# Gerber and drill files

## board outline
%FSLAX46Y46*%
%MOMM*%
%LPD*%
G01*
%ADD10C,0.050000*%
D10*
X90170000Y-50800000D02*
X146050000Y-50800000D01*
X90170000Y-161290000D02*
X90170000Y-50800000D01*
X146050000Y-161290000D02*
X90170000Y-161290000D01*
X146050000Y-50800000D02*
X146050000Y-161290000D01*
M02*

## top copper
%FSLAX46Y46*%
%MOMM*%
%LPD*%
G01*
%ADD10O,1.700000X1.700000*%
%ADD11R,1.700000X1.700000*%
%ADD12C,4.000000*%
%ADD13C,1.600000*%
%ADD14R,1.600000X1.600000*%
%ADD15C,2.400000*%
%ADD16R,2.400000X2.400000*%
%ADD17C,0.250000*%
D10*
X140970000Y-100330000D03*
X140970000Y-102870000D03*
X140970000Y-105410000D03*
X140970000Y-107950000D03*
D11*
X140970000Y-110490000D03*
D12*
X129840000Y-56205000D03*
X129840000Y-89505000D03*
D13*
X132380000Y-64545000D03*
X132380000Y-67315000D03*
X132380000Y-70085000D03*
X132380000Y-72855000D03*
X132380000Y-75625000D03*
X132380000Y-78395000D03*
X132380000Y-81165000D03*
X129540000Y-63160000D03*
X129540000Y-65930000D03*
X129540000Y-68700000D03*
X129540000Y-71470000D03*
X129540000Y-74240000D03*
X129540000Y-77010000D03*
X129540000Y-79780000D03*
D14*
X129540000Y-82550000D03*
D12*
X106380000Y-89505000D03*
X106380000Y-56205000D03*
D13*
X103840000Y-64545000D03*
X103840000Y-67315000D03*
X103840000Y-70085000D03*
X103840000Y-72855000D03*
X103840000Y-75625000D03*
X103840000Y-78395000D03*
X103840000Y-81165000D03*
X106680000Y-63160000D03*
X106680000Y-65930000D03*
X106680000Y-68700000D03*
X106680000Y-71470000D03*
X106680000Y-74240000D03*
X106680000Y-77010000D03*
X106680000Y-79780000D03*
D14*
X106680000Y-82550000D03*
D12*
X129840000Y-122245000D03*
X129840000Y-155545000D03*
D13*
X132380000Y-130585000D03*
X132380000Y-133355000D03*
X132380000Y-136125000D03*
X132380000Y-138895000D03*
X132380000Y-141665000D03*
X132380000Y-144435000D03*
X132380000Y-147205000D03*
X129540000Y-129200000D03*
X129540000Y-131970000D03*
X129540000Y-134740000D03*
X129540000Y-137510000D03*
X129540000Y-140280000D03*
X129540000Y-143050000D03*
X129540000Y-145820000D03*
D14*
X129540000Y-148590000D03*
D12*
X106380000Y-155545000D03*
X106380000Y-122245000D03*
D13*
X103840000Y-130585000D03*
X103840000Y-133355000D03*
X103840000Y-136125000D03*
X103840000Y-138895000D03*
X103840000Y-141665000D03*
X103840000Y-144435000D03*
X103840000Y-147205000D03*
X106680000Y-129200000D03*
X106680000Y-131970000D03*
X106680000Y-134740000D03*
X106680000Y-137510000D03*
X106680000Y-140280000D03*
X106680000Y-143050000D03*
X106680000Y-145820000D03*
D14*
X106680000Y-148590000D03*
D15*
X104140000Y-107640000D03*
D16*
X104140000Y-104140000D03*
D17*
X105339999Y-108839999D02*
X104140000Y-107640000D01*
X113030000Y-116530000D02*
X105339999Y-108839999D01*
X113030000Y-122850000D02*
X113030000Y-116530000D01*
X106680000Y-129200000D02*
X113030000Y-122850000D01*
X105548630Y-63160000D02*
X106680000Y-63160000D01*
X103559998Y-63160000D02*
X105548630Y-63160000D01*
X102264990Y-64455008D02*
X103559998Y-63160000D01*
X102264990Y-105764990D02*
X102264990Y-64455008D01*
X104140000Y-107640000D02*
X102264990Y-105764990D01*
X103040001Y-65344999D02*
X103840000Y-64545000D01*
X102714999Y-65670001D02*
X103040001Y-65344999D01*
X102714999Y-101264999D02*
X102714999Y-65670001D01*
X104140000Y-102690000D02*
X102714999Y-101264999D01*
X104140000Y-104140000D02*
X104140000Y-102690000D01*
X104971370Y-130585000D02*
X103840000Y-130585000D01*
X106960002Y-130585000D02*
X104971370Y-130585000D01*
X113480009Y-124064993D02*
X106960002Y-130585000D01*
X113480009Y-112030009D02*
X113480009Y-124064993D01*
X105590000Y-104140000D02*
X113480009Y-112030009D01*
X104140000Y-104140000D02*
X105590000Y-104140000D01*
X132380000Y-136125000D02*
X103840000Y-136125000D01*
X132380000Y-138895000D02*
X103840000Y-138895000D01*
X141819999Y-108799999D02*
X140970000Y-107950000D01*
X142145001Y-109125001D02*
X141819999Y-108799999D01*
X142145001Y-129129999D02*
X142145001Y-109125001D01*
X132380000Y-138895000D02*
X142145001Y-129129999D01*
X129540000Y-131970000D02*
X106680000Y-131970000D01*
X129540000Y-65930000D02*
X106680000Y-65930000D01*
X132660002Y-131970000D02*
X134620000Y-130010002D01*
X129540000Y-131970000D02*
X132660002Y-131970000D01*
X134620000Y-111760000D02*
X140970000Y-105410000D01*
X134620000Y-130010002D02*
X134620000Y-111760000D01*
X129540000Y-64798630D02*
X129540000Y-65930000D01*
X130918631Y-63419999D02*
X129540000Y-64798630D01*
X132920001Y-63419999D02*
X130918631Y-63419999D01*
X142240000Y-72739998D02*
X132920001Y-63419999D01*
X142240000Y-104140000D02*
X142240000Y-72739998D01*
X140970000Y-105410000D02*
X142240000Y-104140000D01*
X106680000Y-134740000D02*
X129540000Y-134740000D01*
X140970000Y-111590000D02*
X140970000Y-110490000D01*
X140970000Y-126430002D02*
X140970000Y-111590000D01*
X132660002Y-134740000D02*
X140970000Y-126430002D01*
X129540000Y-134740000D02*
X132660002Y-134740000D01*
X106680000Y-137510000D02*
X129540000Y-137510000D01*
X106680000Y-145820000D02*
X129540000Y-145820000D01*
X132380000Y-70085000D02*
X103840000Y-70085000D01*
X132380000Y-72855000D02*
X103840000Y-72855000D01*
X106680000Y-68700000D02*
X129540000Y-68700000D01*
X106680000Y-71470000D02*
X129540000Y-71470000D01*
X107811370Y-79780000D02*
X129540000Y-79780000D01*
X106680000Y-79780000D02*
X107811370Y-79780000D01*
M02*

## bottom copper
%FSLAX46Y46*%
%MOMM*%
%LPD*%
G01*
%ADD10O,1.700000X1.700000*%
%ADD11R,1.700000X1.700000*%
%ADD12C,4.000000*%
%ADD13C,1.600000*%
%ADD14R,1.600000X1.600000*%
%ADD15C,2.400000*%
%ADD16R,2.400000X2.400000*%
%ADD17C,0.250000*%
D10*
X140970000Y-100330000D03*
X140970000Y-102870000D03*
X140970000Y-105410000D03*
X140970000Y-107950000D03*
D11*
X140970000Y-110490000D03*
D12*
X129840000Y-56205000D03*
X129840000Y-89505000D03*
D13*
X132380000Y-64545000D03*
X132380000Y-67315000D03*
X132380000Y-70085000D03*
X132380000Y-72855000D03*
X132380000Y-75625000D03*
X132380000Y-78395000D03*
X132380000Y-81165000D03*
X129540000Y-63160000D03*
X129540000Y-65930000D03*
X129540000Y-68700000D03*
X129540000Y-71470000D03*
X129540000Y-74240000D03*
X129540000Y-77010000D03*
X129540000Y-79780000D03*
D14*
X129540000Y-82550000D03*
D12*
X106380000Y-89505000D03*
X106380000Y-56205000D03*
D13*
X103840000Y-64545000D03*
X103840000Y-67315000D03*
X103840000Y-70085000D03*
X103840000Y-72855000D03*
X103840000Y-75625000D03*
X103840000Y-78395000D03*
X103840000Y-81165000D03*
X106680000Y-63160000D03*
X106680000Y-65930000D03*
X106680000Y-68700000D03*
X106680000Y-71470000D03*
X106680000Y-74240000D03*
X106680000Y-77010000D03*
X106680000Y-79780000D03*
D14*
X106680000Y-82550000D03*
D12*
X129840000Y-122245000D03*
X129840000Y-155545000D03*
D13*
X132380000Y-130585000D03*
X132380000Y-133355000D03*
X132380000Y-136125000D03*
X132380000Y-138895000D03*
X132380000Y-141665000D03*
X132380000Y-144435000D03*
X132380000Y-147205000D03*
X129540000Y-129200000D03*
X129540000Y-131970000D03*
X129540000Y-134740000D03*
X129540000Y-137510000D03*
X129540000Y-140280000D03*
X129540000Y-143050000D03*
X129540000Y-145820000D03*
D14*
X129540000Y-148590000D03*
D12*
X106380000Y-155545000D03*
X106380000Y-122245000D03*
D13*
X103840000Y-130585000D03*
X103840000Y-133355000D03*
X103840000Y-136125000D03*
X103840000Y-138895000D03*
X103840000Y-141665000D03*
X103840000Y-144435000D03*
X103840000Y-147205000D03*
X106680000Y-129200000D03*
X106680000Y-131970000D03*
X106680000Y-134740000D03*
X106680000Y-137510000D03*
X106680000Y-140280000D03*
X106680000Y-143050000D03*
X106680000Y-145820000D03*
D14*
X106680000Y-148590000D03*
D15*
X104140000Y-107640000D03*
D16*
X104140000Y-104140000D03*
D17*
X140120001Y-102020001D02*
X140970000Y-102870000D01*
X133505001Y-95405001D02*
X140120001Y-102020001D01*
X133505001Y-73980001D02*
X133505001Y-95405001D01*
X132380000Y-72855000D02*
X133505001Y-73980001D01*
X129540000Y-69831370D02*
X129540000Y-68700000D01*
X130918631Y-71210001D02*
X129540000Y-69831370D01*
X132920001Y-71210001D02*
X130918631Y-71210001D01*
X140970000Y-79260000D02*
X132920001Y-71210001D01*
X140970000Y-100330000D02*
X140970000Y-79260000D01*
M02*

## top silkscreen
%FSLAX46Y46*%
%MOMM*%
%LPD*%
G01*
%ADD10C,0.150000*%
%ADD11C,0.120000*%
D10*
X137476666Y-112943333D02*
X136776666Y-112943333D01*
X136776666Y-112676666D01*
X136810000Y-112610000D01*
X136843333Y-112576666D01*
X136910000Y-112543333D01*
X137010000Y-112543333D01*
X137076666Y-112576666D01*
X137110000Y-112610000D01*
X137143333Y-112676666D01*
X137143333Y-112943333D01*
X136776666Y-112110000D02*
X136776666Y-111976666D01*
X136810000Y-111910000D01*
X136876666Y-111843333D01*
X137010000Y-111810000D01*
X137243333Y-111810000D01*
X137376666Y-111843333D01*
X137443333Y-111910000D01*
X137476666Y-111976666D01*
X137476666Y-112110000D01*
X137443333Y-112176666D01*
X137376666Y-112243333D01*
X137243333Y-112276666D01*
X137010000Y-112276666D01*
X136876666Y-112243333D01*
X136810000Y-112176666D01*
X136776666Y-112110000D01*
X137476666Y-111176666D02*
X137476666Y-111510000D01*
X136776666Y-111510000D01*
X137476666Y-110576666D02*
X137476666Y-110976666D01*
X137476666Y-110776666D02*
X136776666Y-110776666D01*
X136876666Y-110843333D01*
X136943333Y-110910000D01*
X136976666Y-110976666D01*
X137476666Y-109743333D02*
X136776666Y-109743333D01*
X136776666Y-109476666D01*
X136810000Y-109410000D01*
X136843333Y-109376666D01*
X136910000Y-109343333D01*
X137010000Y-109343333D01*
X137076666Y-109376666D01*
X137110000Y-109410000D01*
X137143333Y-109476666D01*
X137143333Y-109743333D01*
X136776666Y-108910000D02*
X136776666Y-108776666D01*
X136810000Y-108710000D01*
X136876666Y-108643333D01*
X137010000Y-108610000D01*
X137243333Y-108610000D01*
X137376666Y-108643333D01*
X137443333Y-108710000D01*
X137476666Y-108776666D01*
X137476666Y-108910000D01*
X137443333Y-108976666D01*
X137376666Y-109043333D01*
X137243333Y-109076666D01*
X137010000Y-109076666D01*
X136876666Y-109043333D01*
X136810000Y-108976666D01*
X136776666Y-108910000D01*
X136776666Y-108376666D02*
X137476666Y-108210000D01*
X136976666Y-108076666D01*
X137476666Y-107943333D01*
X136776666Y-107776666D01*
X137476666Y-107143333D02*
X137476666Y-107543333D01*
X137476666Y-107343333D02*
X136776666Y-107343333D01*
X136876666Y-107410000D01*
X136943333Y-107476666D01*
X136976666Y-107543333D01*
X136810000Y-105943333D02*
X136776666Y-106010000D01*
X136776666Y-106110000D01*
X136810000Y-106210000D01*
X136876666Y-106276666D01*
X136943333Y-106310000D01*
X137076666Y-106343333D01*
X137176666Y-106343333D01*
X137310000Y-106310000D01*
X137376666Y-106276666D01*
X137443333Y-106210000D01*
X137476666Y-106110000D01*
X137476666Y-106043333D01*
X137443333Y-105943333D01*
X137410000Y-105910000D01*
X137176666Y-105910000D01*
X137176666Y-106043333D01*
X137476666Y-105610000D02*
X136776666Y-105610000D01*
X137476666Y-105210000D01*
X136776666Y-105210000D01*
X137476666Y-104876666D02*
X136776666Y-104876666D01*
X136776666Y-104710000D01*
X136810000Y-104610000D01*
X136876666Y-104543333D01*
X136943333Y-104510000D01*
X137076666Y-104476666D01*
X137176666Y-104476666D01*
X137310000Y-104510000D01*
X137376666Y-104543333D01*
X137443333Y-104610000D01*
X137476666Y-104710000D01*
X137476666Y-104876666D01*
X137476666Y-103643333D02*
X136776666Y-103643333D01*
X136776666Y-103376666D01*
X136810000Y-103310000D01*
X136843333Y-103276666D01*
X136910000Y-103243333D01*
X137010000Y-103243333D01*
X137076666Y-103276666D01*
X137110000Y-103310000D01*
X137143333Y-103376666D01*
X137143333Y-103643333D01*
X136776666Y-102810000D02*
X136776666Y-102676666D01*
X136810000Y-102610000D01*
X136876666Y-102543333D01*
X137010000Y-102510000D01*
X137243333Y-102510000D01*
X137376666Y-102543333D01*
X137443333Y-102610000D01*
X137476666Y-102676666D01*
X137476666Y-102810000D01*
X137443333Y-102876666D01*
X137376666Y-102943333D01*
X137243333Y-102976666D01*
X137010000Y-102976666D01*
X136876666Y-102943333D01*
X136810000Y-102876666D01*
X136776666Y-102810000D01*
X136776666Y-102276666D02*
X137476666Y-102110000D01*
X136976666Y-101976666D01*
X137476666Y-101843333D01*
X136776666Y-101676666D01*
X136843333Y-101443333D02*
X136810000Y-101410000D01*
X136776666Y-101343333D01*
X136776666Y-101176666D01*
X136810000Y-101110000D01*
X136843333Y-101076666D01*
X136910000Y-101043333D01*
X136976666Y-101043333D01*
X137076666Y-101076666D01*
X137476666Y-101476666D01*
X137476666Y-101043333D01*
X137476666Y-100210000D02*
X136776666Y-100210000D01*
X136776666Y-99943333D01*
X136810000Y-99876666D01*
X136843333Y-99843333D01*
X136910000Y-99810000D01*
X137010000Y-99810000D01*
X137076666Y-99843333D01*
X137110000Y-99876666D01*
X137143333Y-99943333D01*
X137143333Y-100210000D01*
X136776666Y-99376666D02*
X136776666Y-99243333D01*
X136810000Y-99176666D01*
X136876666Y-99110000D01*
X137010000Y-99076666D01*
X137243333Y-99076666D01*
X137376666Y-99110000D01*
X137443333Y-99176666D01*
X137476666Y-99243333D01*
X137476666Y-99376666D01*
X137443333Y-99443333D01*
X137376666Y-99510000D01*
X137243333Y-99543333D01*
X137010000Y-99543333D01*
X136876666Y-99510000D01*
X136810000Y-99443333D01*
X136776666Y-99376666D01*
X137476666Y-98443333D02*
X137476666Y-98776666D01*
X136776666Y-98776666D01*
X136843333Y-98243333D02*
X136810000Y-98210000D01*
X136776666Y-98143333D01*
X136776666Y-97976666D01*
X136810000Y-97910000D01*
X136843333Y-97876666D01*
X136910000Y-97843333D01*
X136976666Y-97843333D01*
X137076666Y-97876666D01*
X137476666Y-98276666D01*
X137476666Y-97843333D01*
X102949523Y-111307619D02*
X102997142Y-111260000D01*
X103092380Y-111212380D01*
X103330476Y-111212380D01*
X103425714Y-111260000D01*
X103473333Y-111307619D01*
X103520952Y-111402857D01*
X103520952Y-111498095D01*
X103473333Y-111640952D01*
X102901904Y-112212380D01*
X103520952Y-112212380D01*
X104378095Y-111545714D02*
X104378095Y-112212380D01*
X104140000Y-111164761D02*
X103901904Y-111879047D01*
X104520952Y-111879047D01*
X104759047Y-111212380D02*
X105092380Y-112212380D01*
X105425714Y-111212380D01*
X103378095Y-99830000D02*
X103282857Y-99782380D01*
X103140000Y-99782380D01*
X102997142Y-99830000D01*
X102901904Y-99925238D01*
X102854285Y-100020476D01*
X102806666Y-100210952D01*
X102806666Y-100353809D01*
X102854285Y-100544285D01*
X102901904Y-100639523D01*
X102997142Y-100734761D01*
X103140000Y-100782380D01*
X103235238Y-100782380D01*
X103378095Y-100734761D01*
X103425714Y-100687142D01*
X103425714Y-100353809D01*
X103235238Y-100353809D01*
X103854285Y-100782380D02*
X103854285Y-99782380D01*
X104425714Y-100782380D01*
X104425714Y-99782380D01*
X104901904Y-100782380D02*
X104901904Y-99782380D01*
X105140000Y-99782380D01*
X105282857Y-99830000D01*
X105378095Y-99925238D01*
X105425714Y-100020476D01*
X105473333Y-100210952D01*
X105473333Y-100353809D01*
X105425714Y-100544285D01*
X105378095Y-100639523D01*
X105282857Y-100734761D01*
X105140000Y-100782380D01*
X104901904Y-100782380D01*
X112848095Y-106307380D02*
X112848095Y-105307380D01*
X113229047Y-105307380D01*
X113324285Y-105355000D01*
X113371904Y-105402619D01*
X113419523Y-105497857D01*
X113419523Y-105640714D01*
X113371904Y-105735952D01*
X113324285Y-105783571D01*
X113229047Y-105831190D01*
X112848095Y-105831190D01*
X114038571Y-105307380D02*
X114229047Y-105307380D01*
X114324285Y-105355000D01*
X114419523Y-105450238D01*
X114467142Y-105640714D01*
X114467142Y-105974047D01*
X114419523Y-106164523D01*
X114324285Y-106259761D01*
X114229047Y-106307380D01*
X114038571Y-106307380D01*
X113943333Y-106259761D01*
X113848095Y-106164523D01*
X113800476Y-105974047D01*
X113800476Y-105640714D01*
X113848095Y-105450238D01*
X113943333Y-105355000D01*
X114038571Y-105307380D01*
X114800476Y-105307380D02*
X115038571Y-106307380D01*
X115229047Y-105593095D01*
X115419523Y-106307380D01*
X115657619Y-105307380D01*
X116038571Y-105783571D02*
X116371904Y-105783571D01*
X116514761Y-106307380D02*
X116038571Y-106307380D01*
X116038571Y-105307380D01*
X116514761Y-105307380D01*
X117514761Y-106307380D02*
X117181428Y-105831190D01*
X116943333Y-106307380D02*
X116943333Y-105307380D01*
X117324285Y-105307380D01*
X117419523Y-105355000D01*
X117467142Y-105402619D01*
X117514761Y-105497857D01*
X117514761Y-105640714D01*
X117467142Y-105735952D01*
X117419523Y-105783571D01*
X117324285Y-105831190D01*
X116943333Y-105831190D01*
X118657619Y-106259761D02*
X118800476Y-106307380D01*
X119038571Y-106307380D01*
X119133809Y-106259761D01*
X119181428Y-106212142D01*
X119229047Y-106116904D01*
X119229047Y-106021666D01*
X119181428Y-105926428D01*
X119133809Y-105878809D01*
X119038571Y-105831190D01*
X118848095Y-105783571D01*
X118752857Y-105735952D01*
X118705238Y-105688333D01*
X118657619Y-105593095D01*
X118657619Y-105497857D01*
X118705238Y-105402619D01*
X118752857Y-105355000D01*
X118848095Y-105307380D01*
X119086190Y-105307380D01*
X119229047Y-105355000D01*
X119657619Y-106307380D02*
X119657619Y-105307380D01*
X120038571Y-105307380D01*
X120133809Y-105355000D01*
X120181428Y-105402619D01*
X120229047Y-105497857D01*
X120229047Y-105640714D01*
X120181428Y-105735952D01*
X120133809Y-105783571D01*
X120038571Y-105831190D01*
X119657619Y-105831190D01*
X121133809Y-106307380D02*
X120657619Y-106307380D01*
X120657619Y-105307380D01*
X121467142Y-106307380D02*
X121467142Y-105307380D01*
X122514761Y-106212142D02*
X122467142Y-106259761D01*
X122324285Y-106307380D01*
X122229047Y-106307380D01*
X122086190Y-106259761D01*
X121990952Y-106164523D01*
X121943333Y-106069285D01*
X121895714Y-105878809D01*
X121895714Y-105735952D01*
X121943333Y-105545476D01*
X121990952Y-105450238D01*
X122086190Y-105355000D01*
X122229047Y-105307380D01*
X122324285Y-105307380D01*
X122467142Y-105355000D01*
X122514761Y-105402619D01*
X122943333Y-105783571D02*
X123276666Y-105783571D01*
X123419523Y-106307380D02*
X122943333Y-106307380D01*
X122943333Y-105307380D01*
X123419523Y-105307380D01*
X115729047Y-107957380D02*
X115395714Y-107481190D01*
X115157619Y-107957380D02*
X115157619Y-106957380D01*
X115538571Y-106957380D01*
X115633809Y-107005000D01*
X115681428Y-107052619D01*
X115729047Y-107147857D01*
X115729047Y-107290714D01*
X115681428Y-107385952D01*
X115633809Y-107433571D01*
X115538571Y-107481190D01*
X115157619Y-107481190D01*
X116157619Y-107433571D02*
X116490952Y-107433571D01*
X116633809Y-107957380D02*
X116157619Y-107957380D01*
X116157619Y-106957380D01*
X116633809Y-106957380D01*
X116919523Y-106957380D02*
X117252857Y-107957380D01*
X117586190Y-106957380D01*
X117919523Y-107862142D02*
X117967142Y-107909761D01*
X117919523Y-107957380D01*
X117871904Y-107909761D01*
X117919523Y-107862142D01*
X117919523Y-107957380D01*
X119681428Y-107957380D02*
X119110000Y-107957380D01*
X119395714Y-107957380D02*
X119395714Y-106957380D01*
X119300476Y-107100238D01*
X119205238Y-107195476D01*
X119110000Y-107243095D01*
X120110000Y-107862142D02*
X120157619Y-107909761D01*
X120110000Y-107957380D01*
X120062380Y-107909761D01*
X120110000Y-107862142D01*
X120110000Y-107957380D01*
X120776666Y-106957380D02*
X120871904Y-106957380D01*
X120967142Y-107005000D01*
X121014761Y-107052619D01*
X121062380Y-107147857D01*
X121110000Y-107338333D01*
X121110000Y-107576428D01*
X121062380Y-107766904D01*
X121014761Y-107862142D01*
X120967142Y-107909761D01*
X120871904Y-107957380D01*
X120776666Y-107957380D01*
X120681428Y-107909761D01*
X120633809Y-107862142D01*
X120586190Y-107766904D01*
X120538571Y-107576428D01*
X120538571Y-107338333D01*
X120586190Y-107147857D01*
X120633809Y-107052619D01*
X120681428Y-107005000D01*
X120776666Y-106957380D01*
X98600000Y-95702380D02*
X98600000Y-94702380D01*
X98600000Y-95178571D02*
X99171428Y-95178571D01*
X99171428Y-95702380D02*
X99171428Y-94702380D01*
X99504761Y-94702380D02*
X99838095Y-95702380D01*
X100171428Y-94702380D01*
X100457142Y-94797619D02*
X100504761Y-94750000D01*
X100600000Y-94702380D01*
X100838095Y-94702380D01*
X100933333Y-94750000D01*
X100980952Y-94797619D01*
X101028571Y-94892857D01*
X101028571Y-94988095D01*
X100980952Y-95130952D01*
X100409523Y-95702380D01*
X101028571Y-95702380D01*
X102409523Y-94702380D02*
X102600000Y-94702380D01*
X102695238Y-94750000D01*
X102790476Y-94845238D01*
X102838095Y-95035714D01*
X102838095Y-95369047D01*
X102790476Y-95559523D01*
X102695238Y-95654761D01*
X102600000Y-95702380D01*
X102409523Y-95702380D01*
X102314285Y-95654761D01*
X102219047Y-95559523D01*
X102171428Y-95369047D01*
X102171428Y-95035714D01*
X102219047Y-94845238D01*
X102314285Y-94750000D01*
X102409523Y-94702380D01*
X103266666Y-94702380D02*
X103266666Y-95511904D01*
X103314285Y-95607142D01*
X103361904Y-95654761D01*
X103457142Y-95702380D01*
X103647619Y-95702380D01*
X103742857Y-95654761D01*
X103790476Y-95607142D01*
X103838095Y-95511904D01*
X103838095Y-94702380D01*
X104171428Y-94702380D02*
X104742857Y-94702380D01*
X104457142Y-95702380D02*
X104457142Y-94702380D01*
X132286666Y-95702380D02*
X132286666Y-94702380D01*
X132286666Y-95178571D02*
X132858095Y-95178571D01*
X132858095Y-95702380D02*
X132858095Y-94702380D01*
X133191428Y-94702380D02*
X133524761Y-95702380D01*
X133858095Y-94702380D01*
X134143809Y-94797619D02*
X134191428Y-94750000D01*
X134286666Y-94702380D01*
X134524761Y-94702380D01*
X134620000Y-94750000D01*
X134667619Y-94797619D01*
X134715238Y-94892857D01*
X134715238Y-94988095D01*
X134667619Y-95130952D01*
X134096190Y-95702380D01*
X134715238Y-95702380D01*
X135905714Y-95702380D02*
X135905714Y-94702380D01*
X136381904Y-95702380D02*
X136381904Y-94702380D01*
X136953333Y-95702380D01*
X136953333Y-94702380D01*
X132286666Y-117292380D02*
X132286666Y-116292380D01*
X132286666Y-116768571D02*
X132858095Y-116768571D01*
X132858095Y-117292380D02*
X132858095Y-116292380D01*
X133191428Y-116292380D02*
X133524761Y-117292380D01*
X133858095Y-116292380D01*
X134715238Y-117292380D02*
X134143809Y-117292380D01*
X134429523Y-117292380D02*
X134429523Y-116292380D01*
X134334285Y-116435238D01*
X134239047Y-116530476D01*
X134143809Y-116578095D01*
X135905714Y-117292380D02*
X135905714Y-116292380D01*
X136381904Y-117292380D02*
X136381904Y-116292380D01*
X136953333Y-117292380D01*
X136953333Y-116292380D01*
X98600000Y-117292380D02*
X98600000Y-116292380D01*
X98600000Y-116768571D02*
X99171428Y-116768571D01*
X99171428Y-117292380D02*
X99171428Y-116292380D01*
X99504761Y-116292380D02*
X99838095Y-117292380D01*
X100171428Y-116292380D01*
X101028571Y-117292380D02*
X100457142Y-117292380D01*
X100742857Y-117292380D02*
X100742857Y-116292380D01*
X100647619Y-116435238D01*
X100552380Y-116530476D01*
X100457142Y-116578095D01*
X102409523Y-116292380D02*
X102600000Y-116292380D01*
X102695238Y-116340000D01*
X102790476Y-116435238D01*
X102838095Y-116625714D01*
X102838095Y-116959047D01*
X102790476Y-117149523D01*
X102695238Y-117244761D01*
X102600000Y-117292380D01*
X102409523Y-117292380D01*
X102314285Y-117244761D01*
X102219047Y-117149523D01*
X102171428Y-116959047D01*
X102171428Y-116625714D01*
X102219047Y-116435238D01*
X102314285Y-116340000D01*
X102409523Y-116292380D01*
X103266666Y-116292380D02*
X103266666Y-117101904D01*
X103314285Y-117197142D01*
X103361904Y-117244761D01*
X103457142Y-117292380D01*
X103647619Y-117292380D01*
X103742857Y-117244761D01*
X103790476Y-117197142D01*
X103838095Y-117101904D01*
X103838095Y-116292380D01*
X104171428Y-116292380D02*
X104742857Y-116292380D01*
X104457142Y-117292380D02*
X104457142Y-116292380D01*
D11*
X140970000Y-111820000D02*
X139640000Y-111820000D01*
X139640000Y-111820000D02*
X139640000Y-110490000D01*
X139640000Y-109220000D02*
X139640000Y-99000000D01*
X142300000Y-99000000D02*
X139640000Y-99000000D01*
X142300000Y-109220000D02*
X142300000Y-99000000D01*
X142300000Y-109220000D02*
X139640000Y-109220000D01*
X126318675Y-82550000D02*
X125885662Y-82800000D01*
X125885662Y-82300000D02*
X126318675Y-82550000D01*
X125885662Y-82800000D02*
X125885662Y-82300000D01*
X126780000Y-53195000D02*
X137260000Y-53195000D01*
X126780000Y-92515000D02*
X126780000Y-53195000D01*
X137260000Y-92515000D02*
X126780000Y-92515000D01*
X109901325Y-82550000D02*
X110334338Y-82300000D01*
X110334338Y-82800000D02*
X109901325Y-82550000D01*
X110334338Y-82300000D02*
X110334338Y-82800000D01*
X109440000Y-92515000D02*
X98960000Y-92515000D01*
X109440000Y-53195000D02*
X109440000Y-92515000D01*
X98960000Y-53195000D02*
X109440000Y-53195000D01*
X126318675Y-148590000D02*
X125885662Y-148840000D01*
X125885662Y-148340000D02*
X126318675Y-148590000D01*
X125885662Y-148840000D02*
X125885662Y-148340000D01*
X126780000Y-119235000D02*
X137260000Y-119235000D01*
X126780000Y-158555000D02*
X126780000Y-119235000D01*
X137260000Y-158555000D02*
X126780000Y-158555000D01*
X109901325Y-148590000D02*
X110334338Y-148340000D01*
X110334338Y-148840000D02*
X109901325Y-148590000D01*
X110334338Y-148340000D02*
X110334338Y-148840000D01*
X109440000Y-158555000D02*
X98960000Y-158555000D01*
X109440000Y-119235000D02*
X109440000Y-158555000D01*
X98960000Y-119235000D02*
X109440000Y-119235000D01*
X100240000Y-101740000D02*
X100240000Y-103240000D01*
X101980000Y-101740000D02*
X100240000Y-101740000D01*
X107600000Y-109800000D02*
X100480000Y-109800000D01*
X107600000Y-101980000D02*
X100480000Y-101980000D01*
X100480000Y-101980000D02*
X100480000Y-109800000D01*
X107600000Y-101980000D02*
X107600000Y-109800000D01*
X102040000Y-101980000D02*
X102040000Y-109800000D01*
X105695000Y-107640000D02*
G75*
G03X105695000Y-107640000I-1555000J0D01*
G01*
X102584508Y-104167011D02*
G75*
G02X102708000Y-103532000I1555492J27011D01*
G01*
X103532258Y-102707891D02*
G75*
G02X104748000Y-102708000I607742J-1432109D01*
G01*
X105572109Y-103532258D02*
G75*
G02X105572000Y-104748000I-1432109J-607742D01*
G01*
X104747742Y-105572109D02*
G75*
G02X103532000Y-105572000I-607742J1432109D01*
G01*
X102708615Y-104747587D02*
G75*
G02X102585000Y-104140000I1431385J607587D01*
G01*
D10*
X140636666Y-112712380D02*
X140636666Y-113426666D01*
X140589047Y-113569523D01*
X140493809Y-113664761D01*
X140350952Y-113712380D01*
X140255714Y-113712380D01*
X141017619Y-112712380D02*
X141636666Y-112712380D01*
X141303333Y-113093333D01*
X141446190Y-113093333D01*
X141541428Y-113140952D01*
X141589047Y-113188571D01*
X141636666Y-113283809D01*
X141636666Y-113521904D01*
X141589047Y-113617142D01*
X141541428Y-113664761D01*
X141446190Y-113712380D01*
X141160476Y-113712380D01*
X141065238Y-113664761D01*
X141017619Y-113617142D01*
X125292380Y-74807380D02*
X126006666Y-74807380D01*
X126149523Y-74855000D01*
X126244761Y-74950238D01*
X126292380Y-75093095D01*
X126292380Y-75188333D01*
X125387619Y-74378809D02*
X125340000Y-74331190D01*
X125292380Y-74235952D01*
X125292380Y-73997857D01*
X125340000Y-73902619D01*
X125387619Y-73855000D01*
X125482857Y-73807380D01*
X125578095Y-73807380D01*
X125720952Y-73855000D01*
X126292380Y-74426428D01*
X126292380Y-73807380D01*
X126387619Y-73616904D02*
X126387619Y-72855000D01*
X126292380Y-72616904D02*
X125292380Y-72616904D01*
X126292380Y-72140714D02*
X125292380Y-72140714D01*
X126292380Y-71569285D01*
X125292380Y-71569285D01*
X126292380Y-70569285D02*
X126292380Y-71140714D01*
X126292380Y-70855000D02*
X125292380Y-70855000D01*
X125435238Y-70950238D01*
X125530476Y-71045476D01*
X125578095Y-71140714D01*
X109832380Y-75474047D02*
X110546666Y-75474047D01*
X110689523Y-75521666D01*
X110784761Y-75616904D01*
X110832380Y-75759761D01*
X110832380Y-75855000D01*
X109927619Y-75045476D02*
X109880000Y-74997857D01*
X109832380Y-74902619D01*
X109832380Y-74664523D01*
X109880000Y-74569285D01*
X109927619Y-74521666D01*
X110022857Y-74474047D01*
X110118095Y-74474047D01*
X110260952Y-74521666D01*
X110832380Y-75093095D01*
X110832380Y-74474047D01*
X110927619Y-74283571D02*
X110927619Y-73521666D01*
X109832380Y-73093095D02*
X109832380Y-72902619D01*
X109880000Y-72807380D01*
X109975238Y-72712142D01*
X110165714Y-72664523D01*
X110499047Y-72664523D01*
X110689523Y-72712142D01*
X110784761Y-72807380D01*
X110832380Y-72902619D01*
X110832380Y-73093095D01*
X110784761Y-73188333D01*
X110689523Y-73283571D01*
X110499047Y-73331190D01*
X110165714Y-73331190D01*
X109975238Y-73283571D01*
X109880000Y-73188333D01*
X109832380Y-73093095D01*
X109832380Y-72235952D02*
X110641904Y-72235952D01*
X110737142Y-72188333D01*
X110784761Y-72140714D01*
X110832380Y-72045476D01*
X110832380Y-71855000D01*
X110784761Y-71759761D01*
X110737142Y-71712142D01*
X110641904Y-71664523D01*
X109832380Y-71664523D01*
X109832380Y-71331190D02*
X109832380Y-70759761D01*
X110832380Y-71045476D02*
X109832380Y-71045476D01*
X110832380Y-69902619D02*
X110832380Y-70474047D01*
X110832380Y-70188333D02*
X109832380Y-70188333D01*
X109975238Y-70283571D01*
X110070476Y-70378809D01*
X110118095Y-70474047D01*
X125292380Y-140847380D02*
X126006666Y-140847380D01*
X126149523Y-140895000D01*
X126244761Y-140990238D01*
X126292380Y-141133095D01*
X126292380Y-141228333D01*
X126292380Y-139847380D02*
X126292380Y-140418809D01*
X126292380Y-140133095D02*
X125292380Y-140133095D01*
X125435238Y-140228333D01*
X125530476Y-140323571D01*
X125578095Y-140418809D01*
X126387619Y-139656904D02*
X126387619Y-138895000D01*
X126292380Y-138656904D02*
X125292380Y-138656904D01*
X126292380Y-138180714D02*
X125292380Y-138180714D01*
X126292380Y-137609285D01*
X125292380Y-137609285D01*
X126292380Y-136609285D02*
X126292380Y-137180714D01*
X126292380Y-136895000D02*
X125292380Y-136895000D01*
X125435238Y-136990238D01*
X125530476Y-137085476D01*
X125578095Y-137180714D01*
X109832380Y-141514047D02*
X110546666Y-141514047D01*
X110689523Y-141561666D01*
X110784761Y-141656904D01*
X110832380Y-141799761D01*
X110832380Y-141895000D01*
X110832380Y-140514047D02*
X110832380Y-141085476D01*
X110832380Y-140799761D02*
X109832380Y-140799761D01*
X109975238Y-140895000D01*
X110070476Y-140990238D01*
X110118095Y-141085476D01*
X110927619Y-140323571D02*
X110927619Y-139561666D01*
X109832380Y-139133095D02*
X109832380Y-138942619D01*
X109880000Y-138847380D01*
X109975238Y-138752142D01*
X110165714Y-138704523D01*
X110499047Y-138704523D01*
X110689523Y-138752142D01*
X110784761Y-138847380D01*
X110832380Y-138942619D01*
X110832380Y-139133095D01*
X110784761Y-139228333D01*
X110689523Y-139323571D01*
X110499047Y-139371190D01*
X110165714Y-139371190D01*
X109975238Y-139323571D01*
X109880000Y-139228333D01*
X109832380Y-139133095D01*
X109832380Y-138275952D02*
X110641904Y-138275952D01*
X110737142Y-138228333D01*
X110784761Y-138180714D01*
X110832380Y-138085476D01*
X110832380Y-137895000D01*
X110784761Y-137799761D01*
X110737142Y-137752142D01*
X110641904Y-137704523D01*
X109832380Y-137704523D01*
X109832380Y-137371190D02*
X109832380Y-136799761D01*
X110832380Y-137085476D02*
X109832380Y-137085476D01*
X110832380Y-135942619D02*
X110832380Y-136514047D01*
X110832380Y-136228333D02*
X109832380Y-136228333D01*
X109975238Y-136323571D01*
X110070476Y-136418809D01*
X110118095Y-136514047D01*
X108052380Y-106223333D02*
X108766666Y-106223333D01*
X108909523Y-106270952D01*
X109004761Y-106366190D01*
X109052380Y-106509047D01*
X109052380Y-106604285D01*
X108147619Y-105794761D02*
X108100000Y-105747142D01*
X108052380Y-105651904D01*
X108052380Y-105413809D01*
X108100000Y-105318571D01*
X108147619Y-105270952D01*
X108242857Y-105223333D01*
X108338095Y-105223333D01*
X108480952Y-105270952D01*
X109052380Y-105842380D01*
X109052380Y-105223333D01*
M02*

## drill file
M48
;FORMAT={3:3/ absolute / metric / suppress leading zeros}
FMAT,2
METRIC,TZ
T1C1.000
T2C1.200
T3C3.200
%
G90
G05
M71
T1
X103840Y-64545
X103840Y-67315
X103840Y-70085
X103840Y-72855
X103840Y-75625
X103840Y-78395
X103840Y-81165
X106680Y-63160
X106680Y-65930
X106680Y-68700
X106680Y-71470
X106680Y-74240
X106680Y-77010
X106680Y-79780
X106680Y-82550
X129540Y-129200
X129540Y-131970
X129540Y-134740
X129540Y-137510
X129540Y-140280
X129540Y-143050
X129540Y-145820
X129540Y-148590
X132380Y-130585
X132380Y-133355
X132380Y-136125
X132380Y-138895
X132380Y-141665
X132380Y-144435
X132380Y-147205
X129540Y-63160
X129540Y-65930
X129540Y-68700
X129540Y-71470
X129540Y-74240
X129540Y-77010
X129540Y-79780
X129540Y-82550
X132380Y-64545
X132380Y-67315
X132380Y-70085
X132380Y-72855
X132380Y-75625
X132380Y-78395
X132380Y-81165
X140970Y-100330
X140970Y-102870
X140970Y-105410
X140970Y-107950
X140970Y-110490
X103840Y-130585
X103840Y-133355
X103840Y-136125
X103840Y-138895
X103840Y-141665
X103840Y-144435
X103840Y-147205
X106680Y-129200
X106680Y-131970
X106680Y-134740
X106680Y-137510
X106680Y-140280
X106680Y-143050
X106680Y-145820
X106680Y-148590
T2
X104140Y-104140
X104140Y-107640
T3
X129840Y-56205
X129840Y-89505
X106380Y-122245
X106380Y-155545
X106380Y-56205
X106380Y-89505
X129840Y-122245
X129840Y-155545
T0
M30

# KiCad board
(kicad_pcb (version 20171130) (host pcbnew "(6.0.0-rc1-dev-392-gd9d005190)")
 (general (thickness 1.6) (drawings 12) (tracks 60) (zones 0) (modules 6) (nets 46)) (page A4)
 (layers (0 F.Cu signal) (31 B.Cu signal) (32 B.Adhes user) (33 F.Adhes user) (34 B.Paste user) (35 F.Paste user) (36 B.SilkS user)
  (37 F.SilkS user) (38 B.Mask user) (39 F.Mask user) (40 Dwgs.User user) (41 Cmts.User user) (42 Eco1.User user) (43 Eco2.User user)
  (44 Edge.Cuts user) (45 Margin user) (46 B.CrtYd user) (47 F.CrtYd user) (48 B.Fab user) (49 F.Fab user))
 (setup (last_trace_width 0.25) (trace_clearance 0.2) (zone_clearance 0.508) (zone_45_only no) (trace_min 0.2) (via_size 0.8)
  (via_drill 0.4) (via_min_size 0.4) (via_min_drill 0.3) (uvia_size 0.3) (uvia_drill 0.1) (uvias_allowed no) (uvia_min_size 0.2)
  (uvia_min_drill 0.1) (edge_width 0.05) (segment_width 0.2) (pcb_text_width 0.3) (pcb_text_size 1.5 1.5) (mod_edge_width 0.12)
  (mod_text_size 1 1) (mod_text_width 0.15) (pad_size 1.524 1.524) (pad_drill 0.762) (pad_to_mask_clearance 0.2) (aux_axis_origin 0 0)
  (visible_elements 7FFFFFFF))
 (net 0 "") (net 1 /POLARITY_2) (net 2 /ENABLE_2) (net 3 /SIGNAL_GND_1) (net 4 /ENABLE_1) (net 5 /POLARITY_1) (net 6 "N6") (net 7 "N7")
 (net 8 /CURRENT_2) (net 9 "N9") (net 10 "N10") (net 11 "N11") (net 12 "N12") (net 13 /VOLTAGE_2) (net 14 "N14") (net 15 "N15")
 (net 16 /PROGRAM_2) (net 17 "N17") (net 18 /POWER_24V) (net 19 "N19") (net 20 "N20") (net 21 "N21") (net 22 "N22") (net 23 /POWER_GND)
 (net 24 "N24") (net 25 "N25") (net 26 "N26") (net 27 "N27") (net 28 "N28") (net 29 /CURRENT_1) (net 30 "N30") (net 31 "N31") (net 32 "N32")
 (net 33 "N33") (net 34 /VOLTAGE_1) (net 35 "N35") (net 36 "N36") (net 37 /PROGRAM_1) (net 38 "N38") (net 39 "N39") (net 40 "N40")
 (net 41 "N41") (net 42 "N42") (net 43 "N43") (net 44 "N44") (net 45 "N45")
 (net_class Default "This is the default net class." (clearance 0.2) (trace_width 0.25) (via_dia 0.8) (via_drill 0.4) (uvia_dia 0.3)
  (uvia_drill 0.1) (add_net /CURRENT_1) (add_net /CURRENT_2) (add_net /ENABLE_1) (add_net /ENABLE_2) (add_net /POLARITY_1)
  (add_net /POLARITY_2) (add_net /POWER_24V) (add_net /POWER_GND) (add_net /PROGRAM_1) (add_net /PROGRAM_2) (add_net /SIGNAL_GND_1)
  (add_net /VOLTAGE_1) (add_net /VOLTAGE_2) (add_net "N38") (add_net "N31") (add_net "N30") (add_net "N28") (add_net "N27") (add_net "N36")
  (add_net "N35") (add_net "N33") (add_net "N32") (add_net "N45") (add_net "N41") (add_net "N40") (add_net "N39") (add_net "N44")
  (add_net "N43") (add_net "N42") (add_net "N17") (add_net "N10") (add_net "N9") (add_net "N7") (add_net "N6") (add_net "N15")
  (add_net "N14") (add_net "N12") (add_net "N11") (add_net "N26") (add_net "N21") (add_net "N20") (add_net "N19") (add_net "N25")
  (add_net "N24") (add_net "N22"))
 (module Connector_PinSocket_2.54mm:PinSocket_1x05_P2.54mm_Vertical (layer F.Cu) (at 140.97 110.49 180)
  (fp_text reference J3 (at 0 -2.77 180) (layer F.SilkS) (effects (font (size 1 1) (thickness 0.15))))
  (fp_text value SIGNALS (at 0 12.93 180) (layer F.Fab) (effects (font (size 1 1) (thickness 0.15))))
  (fp_line (start 0 -1.33) (end 1.33 -1.33) (layer F.SilkS) (width 0.12))
  (fp_line (start 1.33 -1.33) (end 1.33 0) (layer F.SilkS) (width 0.12))
  (fp_line (start 1.33 1.27) (end 1.33 11.49) (layer F.SilkS) (width 0.12))
  (fp_line (start -1.33 11.49) (end 1.33 11.49) (layer F.SilkS) (width 0.12))
  (fp_line (start -1.33 1.27) (end -1.33 11.49) (layer F.SilkS) (width 0.12))
  (fp_line (start -1.33 1.27) (end 1.33 1.27) (layer F.SilkS) (width 0.12))
  (pad 5 thru_hole oval (at 0 10.16 180) (size 1.7 1.7) (drill 1) (layers *.Cu *.Mask) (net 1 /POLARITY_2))
  (pad 4 thru_hole oval (at 0 7.62 180) (size 1.7 1.7) (drill 1) (layers *.Cu *.Mask) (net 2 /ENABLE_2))
  (pad 3 thru_hole oval (at 0 5.08 180) (size 1.7 1.7) (drill 1) (layers *.Cu *.Mask) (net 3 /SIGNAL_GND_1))
  (pad 2 thru_hole oval (at 0 2.54 180) (size 1.7 1.7) (drill 1) (layers *.Cu *.Mask) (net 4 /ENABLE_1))
  (pad 1 thru_hole rect (at 0 0 180) (size 1.7 1.7) (drill 1) (layers *.Cu *.Mask) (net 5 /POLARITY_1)))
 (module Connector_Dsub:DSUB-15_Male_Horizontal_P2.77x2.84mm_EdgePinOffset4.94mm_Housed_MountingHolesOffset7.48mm (layer F.Cu)
  (at 129.54 82.55 90)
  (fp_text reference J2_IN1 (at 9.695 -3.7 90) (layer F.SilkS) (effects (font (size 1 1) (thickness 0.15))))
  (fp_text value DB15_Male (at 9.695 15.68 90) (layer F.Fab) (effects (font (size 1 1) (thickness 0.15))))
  (fp_line (start 0 -3.221325) (end -0.25 -3.654338) (layer F.SilkS) (width 0.12))
  (fp_line (start 0.25 -3.654338) (end 0 -3.221325) (layer F.SilkS) (width 0.12))
  (fp_line (start -0.25 -3.654338) (end 0.25 -3.654338) (layer F.SilkS) (width 0.12))
  (fp_line (start 29.355 -2.76) (end 29.355 7.72) (layer F.SilkS) (width 0.12))
  (fp_line (start -9.965 -2.76) (end 29.355 -2.76) (layer F.SilkS) (width 0.12))
  (fp_line (start -9.965 7.72) (end -9.965 -2.76) (layer F.SilkS) (width 0.12))
  (pad 0 thru_hole circle (at 26.345 0.3 90) (size 4 4) (drill 3.2) (layers *.Cu *.Mask))
  (pad 0 thru_hole circle (at -6.955 0.3 90) (size 4 4) (drill 3.2) (layers *.Cu *.Mask))
  (pad 15 thru_hole circle (at 18.005 2.84 90) (size 1.6 1.6) (drill 1) (layers *.Cu *.Mask) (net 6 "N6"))
  (pad 14 thru_hole circle (at 15.235 2.84 90) (size 1.6 1.6) (drill 1) (layers *.Cu *.Mask) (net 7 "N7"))
  (pad 13 thru_hole circle (at 12.465 2.84 90) (size 1.6 1.6) (drill 1) (layers *.Cu *.Mask) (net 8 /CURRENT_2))
  (pad 12 thru_hole circle (at 9.695 2.84 90) (size 1.6 1.6) (drill 1) (layers *.Cu *.Mask) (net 2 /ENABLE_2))
  (pad 11 thru_hole circle (at 6.925 2.84 90) (size 1.6 1.6) (drill 1) (layers *.Cu *.Mask) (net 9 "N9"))
  (pad 10 thru_hole circle (at 4.155 2.84 90) (size 1.6 1.6) (drill 1) (layers *.Cu *.Mask) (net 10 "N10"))
  (pad 9 thru_hole circle (at 1.385 2.84 90) (size 1.6 1.6) (drill 1) (layers *.Cu *.Mask) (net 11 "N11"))
  (pad 8 thru_hole circle (at 19.39 0 90) (size 1.6 1.6) (drill 1) (layers *.Cu *.Mask) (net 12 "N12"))
  (pad 7 thru_hole circle (at 16.62 0 90) (size 1.6 1.6) (drill 1) (layers *.Cu *.Mask) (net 3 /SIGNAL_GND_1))
  (pad 6 thru_hole circle (at 13.85 0 90) (size 1.6 1.6) (drill 1) (layers *.Cu *.Mask) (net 1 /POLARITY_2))
  (pad 5 thru_hole circle (at 11.08 0 90) (size 1.6 1.6) (drill 1) (layers *.Cu *.Mask) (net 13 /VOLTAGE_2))
  (pad 4 thru_hole circle (at 8.31 0 90) (size 1.6 1.6) (drill 1) (layers *.Cu *.Mask) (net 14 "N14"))
  (pad 3 thru_hole circle (at 5.54 0 90) (size 1.6 1.6) (drill 1) (layers *.Cu *.Mask) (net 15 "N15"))
  (pad 2 thru_hole circle (at 2.77 0 90) (size 1.6 1.6) (drill 1) (layers *.Cu *.Mask) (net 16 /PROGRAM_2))
  (pad 1 thru_hole rect (at 0 0 90) (size 1.6 1.6) (drill 1) (layers *.Cu *.Mask) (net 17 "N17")))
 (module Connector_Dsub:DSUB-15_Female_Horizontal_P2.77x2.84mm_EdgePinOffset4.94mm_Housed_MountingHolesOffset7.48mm (layer F.Cu)
  (at 106.68 82.55 270)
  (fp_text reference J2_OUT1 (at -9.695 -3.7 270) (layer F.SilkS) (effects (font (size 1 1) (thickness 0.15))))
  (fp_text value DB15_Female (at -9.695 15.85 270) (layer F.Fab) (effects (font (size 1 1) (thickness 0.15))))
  (fp_line (start 0 -3.221325) (end -0.25 -3.654338) (layer F.SilkS) (width 0.12))
  (fp_line (start 0.25 -3.654338) (end 0 -3.221325) (layer F.SilkS) (width 0.12))
  (fp_line (start -0.25 -3.654338) (end 0.25 -3.654338) (layer F.SilkS) (width 0.12))
  (fp_line (start 9.965 -2.76) (end 9.965 7.72) (layer F.SilkS) (width 0.12))
  (fp_line (start -29.355 -2.76) (end 9.965 -2.76) (layer F.SilkS) (width 0.12))
  (fp_line (start -29.355 7.72) (end -29.355 -2.76) (layer F.SilkS) (width 0.12))
  (pad 0 thru_hole circle (at 6.955 0.3 270) (size 4 4) (drill 3.2) (layers *.Cu *.Mask))
  (pad 0 thru_hole circle (at -26.345 0.3 270) (size 4 4) (drill 3.2) (layers *.Cu *.Mask))
  (pad 15 thru_hole circle (at -18.005 2.84 270) (size 1.6 1.6) (drill 1) (layers *.Cu *.Mask) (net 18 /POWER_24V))
  (pad 14 thru_hole circle (at -15.235 2.84 270) (size 1.6 1.6) (drill 1) (layers *.Cu *.Mask) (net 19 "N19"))
  (pad 13 thru_hole circle (at -12.465 2.84 270) (size 1.6 1.6) (drill 1) (layers *.Cu *.Mask) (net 8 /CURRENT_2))
  (pad 12 thru_hole circle (at -9.695 2.84 270) (size 1.6 1.6) (drill 1) (layers *.Cu *.Mask) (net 2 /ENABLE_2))
  (pad 11 thru_hole circle (at -6.925 2.84 270) (size 1.6 1.6) (drill 1) (layers *.Cu *.Mask) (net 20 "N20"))
  (pad 10 thru_hole circle (at -4.155 2.84 270) (size 1.6 1.6) (drill 1) (layers *.Cu *.Mask) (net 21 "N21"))
  (pad 9 thru_hole circle (at -1.385 2.84 270) (size 1.6 1.6) (drill 1) (layers *.Cu *.Mask) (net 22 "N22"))
  (pad 8 thru_hole circle (at -19.39 0 270) (size 1.6 1.6) (drill 1) (layers *.Cu *.Mask) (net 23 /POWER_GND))
  (pad 7 thru_hole circle (at -16.62 0 270) (size 1.6 1.6) (drill 1) (layers *.Cu *.Mask) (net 3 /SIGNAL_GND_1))
  (pad 6 thru_hole circle (at -13.85 0 270) (size 1.6 1.6) (drill 1) (layers *.Cu *.Mask) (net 1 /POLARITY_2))
  (pad 5 thru_hole circle (at -11.08 0 270) (size 1.6 1.6) (drill 1) (layers *.Cu *.Mask) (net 13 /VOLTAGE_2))
  (pad 4 thru_hole circle (at -8.31 0 270) (size 1.6 1.6) (drill 1) (layers *.Cu *.Mask) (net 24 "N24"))
  (pad 3 thru_hole circle (at -5.54 0 270) (size 1.6 1.6) (drill 1) (layers *.Cu *.Mask) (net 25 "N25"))
  (pad 2 thru_hole circle (at -2.77 0 270) (size 1.6 1.6) (drill 1) (layers *.Cu *.Mask) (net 16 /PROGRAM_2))
  (pad 1 thru_hole rect (at 0 0 270) (size 1.6 1.6) (drill 1) (layers *.Cu *.Mask) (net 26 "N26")))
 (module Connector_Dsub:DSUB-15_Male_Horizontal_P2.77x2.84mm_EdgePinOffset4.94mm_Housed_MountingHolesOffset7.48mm (layer F.Cu)
  (at 129.54 148.59 90)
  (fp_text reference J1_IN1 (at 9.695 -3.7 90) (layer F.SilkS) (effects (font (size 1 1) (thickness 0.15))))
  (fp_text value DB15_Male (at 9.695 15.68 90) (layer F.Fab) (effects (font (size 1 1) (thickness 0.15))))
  (fp_line (start 0 -3.221325) (end -0.25 -3.654338) (layer F.SilkS) (width 0.12))
  (fp_line (start 0.25 -3.654338) (end 0 -3.221325) (layer F.SilkS) (width 0.12))
  (fp_line (start -0.25 -3.654338) (end 0.25 -3.654338) (layer F.SilkS) (width 0.12))
  (fp_line (start 29.355 -2.76) (end 29.355 7.72) (layer F.SilkS) (width 0.12))
  (fp_line (start -9.965 -2.76) (end 29.355 -2.76) (layer F.SilkS) (width 0.12))
  (fp_line (start -9.965 7.72) (end -9.965 -2.76) (layer F.SilkS) (width 0.12))
  (pad 0 thru_hole circle (at 26.345 0.3 90) (size 4 4) (drill 3.2) (layers *.Cu *.Mask))
  (pad 0 thru_hole circle (at -6.955 0.3 90) (size 4 4) (drill 3.2) (layers *.Cu *.Mask))
  (pad 15 thru_hole circle (at 18.005 2.84 90) (size 1.6 1.6) (drill 1) (layers *.Cu *.Mask) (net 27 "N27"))
  (pad 14 thru_hole circle (at 15.235 2.84 90) (size 1.6 1.6) (drill 1) (layers *.Cu *.Mask) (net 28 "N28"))
  (pad 13 thru_hole circle (at 12.465 2.84 90) (size 1.6 1.6) (drill 1) (layers *.Cu *.Mask) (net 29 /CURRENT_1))
  (pad 12 thru_hole circle (at 9.695 2.84 90) (size 1.6 1.6) (drill 1) (layers *.Cu *.Mask) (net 4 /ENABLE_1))
  (pad 11 thru_hole circle (at 6.925 2.84 90) (size 1.6 1.6) (drill 1) (layers *.Cu *.Mask) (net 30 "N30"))
  (pad 10 thru_hole circle (at 4.155 2.84 90) (size 1.6 1.6) (drill 1) (layers *.Cu *.Mask) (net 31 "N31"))
  (pad 9 thru_hole circle (at 1.385 2.84 90) (size 1.6 1.6) (drill 1) (layers *.Cu *.Mask) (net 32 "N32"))
  (pad 8 thru_hole circle (at 19.39 0 90) (size 1.6 1.6) (drill 1) (layers *.Cu *.Mask) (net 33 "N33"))
  (pad 7 thru_hole circle (at 16.62 0 90) (size 1.6 1.6) (drill 1) (layers *.Cu *.Mask) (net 3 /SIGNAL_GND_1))
  (pad 6 thru_hole circle (at 13.85 0 90) (size 1.6 1.6) (drill 1) (layers *.Cu *.Mask) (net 5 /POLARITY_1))
  (pad 5 thru_hole circle (at 11.08 0 90) (size 1.6 1.6) (drill 1) (layers *.Cu *.Mask) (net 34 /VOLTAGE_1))
  (pad 4 thru_hole circle (at 8.31 0 90) (size 1.6 1.6) (drill 1) (layers *.Cu *.Mask) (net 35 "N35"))
  (pad 3 thru_hole circle (at 5.54 0 90) (size 1.6 1.6) (drill 1) (layers *.Cu *.Mask) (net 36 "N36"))
  (pad 2 thru_hole circle (at 2.77 0 90) (size 1.6 1.6) (drill 1) (layers *.Cu *.Mask) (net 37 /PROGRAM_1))
  (pad 1 thru_hole rect (at 0 0 90) (size 1.6 1.6) (drill 1) (layers *.Cu *.Mask) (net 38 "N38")))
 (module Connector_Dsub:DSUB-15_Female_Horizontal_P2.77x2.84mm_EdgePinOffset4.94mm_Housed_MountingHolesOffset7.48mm (layer F.Cu)
  (at 106.68 148.59 270)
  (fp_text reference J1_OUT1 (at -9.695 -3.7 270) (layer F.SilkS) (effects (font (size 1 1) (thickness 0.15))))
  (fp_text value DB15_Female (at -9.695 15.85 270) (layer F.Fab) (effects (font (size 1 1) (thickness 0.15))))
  (fp_line (start 0 -3.221325) (end -0.25 -3.654338) (layer F.SilkS) (width 0.12))
  (fp_line (start 0.25 -3.654338) (end 0 -3.221325) (layer F.SilkS) (width 0.12))
  (fp_line (start -0.25 -3.654338) (end 0.25 -3.654338) (layer F.SilkS) (width 0.12))
  (fp_line (start 9.965 -2.76) (end 9.965 7.72) (layer F.SilkS) (width 0.12))
  (fp_line (start -29.355 -2.76) (end 9.965 -2.76) (layer F.SilkS) (width 0.12))
  (fp_line (start -29.355 7.72) (end -29.355 -2.76) (layer F.SilkS) (width 0.12))
  (pad 0 thru_hole circle (at 6.955 0.3 270) (size 4 4) (drill 3.2) (layers *.Cu *.Mask))
  (pad 0 thru_hole circle (at -26.345 0.3 270) (size 4 4) (drill 3.2) (layers *.Cu *.Mask))
  (pad 15 thru_hole circle (at -18.005 2.84 270) (size 1.6 1.6) (drill 1) (layers *.Cu *.Mask) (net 18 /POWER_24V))
  (pad 14 thru_hole circle (at -15.235 2.84 270) (size 1.6 1.6) (drill 1) (layers *.Cu *.Mask) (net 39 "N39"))
  (pad 13 thru_hole circle (at -12.465 2.84 270) (size 1.6 1.6) (drill 1) (layers *.Cu *.Mask) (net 29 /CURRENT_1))
  (pad 12 thru_hole circle (at -9.695 2.84 270) (size 1.6 1.6) (drill 1) (layers *.Cu *.Mask) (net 4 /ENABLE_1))
  (pad 11 thru_hole circle (at -6.925 2.84 270) (size 1.6 1.6) (drill 1) (layers *.Cu *.Mask) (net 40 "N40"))
  (pad 10 thru_hole circle (at -4.155 2.84 270) (size 1.6 1.6) (drill 1) (layers *.Cu *.Mask) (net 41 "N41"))
  (pad 9 thru_hole circle (at -1.385 2.84 270) (size 1.6 1.6) (drill 1) (layers *.Cu *.Mask) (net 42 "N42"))
  (pad 8 thru_hole circle (at -19.39 0 270) (size 1.6 1.6) (drill 1) (layers *.Cu *.Mask) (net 23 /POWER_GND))
  (pad 7 thru_hole circle (at -16.62 0 270) (size 1.6 1.6) (drill 1) (layers *.Cu *.Mask) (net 3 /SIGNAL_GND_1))
  (pad 6 thru_hole circle (at -13.85 0 270) (size 1.6 1.6) (drill 1) (layers *.Cu *.Mask) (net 5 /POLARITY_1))
  (pad 5 thru_hole circle (at -11.08 0 270) (size 1.6 1.6) (drill 1) (layers *.Cu *.Mask) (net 34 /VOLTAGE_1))
  (pad 4 thru_hole circle (at -8.31 0 270) (size 1.6 1.6) (drill 1) (layers *.Cu *.Mask) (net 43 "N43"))
  (pad 3 thru_hole circle (at -5.54 0 270) (size 1.6 1.6) (drill 1) (layers *.Cu *.Mask) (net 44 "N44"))
  (pad 2 thru_hole circle (at -2.77 0 270) (size 1.6 1.6) (drill 1) (layers *.Cu *.Mask) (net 37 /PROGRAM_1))
  (pad 1 thru_hole rect (at 0 0 270) (size 1.6 1.6) (drill 1) (layers *.Cu *.Mask) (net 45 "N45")))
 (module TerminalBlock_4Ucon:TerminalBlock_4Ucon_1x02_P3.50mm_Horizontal (layer F.Cu) (at 104.14 104.14 270)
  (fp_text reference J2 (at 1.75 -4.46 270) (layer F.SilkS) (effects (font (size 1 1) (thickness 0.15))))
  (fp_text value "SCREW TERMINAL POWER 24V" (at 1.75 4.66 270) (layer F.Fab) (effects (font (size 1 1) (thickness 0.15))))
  (fp_line (start -2.4 3.9) (end -0.9 3.9) (layer F.SilkS) (width 0.12))
  (fp_line (start -2.4 2.16) (end -2.4 3.9) (layer F.SilkS) (width 0.12))
  (fp_line (start 5.66 -3.46) (end 5.66 3.66) (layer F.SilkS) (width 0.12))
  (fp_line (start -2.16 -3.46) (end -2.16 3.66) (layer F.SilkS) (width 0.12))
  (fp_line (start -2.16 3.66) (end 5.66 3.66) (layer F.SilkS) (width 0.12))
  (fp_line (start -2.16 -3.46) (end 5.66 -3.46) (layer F.SilkS) (width 0.12))
  (fp_line (start -2.16 2.1) (end 5.66 2.1) (layer F.SilkS) (width 0.12))
  (fp_circle (center 3.5 0) (end 5.055 0) (layer F.SilkS) (width 0.12))
  (fp_arc (start 0 0) (end -0.608 1.432) (angle -24) (layer F.SilkS) (width 0.12))
  (fp_arc (start 0 0) (end -1.432 -0.608) (angle -46) (layer F.SilkS) (width 0.12))
  (fp_arc (start 0 0) (end 0.608 -1.432) (angle -46) (layer F.SilkS) (width 0.12))
  (fp_arc (start 0 0) (end 1.432 0.608) (angle -46) (layer F.SilkS) (width 0.12))
  (fp_arc (start 0 0) (end 0 1.555) (angle -23) (layer F.SilkS) (width 0.12))
  (pad 2 thru_hole circle (at 3.5 0 270) (size 2.4 2.4) (drill 1.2) (layers *.Cu *.Mask) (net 23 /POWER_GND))
  (pad 1 thru_hole rect (at 0 0 270) (size 2.4 2.4) (drill 1.2) (layers *.Cu *.Mask) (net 18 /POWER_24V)))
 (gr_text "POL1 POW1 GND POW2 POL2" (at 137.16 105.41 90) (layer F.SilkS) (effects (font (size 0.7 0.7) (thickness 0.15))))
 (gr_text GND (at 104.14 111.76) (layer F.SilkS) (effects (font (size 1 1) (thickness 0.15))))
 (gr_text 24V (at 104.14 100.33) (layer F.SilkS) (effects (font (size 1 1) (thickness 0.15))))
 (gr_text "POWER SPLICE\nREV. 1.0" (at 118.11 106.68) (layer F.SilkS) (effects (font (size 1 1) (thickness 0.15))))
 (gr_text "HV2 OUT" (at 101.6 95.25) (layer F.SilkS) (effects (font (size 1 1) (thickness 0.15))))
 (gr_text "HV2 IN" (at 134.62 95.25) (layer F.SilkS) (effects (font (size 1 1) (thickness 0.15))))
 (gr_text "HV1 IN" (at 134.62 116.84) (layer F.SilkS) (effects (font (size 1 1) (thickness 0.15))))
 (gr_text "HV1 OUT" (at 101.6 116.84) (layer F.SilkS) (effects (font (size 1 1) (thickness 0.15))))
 (gr_line (start 90.17 50.8) (end 146.05 50.8) (layer Edge.Cuts) (width 0.05))
 (gr_line (start 90.17 161.29) (end 90.17 50.8) (layer Edge.Cuts) (width 0.05))
 (gr_line (start 146.05 161.29) (end 90.17 161.29) (layer Edge.Cuts) (width 0.05))
 (gr_line (start 146.05 50.8) (end 146.05 161.29) (layer Edge.Cuts) (width 0.05))
 (segment (start 105.339999 108.839999) (end 104.14 107.64) (width 0.25) (layer F.Cu) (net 23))
 (segment (start 113.03 116.53) (end 105.339999 108.839999) (width 0.25) (layer F.Cu) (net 23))
 (segment (start 113.03 122.85) (end 113.03 116.53) (width 0.25) (layer F.Cu) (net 23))
 (segment (start 106.68 129.2) (end 113.03 122.85) (width 0.25) (layer F.Cu) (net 23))
 (segment (start 105.54863 63.16) (end 106.68 63.16) (width 0.25) (layer F.Cu) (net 23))
 (segment (start 103.559998 63.16) (end 105.54863 63.16) (width 0.25) (layer F.Cu) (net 23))
 (segment (start 102.26499 64.455008) (end 103.559998 63.16) (width 0.25) (layer F.Cu) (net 23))
 (segment (start 102.26499 105.76499) (end 102.26499 64.455008) (width 0.25) (layer F.Cu) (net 23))
 (segment (start 104.14 107.64) (end 102.26499 105.76499) (width 0.25) (layer F.Cu) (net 23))
 (segment (start 103.040001 65.344999) (end 103.84 64.545) (width 0.25) (layer F.Cu) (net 18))
 (segment (start 102.714999 65.670001) (end 103.040001 65.344999) (width 0.25) (layer F.Cu) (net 18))
 (segment (start 102.714999 101.264999) (end 102.714999 65.670001) (width 0.25) (layer F.Cu) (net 18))
 (segment (start 104.14 102.69) (end 102.714999 101.264999) (width 0.25) (layer F.Cu) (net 18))
 (segment (start 104.14 104.14) (end 104.14 102.69) (width 0.25) (layer F.Cu) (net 18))
 (segment (start 104.97137 130.585) (end 103.84 130.585) (width 0.25) (layer F.Cu) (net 18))
 (segment (start 106.960002 130.585) (end 104.97137 130.585) (width 0.25) (layer F.Cu) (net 18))
 (segment (start 113.480009 124.064993) (end 106.960002 130.585) (width 0.25) (layer F.Cu) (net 18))
 (segment (start 113.480009 112.030009) (end 113.480009 124.064993) (width 0.25) (layer F.Cu) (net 18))
 (segment (start 105.59 104.14) (end 113.480009 112.030009) (width 0.25) (layer F.Cu) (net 18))
 (segment (start 104.14 104.14) (end 105.59 104.14) (width 0.25) (layer F.Cu) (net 18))
 (segment (start 132.38 136.125) (end 103.84 136.125) (width 0.25) (layer F.Cu) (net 29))
 (segment (start 132.38 138.895) (end 103.84 138.895) (width 0.25) (layer F.Cu) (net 4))
 (segment (start 141.819999 108.799999) (end 140.97 107.95) (width 0.25) (layer F.Cu) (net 4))
 (segment (start 142.145001 109.125001) (end 141.819999 108.799999) (width 0.25) (layer F.Cu) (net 4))
 (segment (start 142.145001 129.129999) (end 142.145001 109.125001) (width 0.25) (layer F.Cu) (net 4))
 (segment (start 132.38 138.895) (end 142.145001 129.129999) (width 0.25) (layer F.Cu) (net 4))
 (segment (start 129.54 131.97) (end 106.68 131.97) (width 0.25) (layer F.Cu) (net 3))
 (segment (start 129.54 65.93) (end 106.68 65.93) (width 0.25) (layer F.Cu) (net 3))
 (segment (start 132.660002 131.97) (end 134.62 130.010002) (width 0.25) (layer F.Cu) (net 3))
 (segment (start 129.54 131.97) (end 132.660002 131.97) (width 0.25) (layer F.Cu) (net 3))
 (segment (start 134.62 111.76) (end 140.97 105.41) (width 0.25) (layer F.Cu) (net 3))
 (segment (start 134.62 130.010002) (end 134.62 111.76) (width 0.25) (layer F.Cu) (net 3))
 (segment (start 129.54 64.79863) (end 129.54 65.93) (width 0.25) (layer F.Cu) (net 3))
 (segment (start 130.918631 63.419999) (end 129.54 64.79863) (width 0.25) (layer F.Cu) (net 3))
 (segment (start 132.920001 63.419999) (end 130.918631 63.419999) (width 0.25) (layer F.Cu) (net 3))
 (segment (start 142.24 72.739998) (end 132.920001 63.419999) (width 0.25) (layer F.Cu) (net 3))
 (segment (start 142.24 104.14) (end 142.24 72.739998) (width 0.25) (layer F.Cu) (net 3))
 (segment (start 140.97 105.41) (end 142.24 104.14) (width 0.25) (layer F.Cu) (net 3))
 (segment (start 106.68 134.74) (end 129.54 134.74) (width 0.25) (layer F.Cu) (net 5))
 (segment (start 140.97 111.59) (end 140.97 110.49) (width 0.25) (layer F.Cu) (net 5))
 (segment (start 140.97 126.430002) (end 140.97 111.59) (width 0.25) (layer F.Cu) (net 5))
 (segment (start 132.660002 134.74) (end 140.97 126.430002) (width 0.25) (layer F.Cu) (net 5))
 (segment (start 129.54 134.74) (end 132.660002 134.74) (width 0.25) (layer F.Cu) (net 5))
 (segment (start 106.68 137.51) (end 129.54 137.51) (width 0.25) (layer F.Cu) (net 34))
 (segment (start 106.68 145.82) (end 129.54 145.82) (width 0.25) (layer F.Cu) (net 37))
 (segment (start 132.38 70.085) (end 103.84 70.085) (width 0.25) (layer F.Cu) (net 8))
 (segment (start 132.38 72.855) (end 103.84 72.855) (width 0.25) (layer F.Cu) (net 2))
 (segment (start 140.120001 102.020001) (end 140.97 102.87) (width 0.25) (layer B.Cu) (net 2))
 (segment (start 133.505001 95.405001) (end 140.120001 102.020001) (width 0.25) (layer B.Cu) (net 2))
 (segment (start 133.505001 73.980001) (end 133.505001 95.405001) (width 0.25) (layer B.Cu) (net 2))
 (segment (start 132.38 72.855) (end 133.505001 73.980001) (width 0.25) (layer B.Cu) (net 2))
 (segment (start 106.68 68.7) (end 129.54 68.7) (width 0.25) (layer F.Cu) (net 1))
 (segment (start 129.54 69.83137) (end 129.54 68.7) (width 0.25) (layer B.Cu) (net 1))
 (segment (start 130.918631 71.210001) (end 129.54 69.83137) (width 0.25) (layer B.Cu) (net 1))
 (segment (start 132.920001 71.210001) (end 130.918631 71.210001) (width 0.25) (layer B.Cu) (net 1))
 (segment (start 140.97 79.26) (end 132.920001 71.210001) (width 0.25) (layer B.Cu) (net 1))
 (segment (start 140.97 100.33) (end 140.97 79.26) (width 0.25) (layer B.Cu) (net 1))
 (segment (start 106.68 71.47) (end 129.54 71.47) (width 0.25) (layer F.Cu) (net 13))
 (segment (start 107.81137 79.78) (end 129.54 79.78) (width 0.25) (layer F.Cu) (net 16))
 (segment (start 106.68 79.78) (end 107.81137 79.78) (width 0.25) (layer F.Cu) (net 16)))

